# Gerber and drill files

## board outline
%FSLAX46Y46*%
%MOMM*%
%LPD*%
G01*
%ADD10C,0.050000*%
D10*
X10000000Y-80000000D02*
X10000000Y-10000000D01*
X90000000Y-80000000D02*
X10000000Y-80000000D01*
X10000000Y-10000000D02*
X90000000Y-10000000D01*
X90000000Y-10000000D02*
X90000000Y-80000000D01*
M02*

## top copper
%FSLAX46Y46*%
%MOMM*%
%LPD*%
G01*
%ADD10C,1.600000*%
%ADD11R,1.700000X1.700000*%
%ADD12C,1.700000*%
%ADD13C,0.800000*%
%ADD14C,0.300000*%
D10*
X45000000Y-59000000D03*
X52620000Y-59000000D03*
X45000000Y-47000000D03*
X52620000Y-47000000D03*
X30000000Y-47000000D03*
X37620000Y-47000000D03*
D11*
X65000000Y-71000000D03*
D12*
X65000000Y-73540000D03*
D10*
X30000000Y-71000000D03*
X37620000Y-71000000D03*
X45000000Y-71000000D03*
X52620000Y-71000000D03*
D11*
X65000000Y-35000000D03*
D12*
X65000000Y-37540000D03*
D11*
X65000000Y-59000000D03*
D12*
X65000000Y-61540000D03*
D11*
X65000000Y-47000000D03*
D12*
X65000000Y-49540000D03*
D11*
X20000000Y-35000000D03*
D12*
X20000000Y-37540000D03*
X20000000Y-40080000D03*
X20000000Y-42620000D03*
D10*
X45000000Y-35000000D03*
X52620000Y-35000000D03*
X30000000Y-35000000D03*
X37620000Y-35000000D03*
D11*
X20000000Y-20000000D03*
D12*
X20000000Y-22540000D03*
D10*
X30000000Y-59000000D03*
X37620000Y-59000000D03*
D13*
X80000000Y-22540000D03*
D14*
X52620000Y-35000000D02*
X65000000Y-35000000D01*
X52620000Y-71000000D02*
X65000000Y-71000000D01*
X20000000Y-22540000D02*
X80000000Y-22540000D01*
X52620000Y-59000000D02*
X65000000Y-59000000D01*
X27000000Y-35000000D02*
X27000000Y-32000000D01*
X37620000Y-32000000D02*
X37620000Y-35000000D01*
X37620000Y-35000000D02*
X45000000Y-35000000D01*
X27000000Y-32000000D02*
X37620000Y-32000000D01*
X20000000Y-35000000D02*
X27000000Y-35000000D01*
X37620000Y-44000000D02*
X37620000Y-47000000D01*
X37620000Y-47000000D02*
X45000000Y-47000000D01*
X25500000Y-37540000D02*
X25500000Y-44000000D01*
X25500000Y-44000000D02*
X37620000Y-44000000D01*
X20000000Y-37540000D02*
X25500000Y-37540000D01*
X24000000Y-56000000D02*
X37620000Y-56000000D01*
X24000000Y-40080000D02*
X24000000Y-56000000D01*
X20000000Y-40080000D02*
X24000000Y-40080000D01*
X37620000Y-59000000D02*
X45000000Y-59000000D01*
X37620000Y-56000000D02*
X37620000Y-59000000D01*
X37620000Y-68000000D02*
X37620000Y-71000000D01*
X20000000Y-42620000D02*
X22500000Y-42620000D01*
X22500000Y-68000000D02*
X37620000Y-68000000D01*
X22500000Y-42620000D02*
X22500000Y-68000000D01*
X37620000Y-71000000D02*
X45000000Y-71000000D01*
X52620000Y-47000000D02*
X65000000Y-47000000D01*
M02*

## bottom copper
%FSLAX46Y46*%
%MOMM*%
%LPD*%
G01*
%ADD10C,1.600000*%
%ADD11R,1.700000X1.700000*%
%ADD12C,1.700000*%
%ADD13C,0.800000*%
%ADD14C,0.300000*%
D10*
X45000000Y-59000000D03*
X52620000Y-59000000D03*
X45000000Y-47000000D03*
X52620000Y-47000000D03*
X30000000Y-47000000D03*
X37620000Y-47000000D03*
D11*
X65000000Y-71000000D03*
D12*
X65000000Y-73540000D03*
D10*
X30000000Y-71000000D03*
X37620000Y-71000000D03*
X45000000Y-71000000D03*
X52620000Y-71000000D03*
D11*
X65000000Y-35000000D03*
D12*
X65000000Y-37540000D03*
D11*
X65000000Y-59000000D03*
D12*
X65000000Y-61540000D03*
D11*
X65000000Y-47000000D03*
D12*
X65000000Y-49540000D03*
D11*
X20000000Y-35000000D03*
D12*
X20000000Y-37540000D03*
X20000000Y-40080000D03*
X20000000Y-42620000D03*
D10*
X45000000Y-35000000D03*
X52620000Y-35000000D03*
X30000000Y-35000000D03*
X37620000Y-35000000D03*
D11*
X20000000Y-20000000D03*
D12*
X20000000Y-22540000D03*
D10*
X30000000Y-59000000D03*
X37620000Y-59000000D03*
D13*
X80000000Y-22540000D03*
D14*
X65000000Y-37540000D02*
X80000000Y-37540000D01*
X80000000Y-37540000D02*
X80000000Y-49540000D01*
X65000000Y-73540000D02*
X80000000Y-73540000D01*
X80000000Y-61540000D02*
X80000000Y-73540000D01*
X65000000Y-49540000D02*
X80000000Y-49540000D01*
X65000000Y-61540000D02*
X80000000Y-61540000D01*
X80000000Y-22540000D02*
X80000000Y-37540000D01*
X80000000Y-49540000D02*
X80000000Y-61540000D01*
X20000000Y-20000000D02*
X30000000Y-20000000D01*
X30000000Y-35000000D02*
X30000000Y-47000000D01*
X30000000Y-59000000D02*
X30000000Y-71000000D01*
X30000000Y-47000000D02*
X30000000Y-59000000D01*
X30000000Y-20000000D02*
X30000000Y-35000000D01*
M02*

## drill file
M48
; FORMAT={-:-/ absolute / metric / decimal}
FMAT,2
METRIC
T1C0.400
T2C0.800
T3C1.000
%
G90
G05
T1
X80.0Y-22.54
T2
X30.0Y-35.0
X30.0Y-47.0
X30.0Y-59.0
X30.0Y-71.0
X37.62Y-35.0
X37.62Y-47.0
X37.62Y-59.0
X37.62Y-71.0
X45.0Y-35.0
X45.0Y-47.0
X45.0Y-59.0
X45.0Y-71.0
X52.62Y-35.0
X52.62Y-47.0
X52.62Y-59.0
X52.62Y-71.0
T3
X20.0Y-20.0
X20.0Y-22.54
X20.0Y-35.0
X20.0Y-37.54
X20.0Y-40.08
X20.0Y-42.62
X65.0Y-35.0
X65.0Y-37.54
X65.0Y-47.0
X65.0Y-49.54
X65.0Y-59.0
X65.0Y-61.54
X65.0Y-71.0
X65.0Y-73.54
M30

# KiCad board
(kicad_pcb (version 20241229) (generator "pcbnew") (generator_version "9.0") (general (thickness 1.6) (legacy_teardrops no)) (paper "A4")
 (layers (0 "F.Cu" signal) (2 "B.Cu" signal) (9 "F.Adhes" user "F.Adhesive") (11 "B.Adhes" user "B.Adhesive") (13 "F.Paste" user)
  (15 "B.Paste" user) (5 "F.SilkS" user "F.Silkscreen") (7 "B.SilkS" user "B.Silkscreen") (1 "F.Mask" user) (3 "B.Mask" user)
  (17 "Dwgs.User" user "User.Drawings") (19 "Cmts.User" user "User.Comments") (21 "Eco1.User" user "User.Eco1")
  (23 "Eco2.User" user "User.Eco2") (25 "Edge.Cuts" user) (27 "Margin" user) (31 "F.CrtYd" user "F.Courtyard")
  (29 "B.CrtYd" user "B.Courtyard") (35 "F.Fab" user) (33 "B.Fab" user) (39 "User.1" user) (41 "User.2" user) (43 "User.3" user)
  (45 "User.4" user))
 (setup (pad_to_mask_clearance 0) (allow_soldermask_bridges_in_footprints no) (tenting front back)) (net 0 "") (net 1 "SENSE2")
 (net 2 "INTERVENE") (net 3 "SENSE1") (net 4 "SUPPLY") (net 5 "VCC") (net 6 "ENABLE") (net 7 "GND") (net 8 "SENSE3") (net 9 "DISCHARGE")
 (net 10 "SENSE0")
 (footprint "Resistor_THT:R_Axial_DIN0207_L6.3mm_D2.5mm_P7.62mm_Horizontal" (layer "F.Cu") (at 45 59)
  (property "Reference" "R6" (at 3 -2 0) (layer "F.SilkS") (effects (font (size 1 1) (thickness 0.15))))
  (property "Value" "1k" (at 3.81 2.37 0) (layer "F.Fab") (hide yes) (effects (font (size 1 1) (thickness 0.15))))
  (pad "1" thru_hole circle (at 0 0) (size 1.6 1.6) (drill 0.8) (layers "*.Cu" "*.Mask") (remove_unused_layers no) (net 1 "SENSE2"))
  (pad "2" thru_hole circle (at 7.62 0) (size 1.6 1.6) (drill 0.8) (layers "*.Cu" "*.Mask") (remove_unused_layers no) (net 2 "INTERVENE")))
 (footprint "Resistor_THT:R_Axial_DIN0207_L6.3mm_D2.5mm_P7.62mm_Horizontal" (layer "F.Cu") (at 45 47)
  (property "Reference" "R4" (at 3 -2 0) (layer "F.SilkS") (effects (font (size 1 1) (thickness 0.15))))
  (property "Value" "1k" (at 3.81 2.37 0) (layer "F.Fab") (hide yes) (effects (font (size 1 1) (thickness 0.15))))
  (pad "1" thru_hole circle (at 0 0) (size 1.6 1.6) (drill 0.8) (layers "*.Cu" "*.Mask") (remove_unused_layers no) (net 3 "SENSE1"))
  (pad "2" thru_hole circle (at 7.62 0) (size 1.6 1.6) (drill 0.8) (layers "*.Cu" "*.Mask") (remove_unused_layers no) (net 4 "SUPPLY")))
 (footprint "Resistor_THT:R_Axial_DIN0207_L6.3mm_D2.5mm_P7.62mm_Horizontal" (layer "F.Cu") (at 30 47)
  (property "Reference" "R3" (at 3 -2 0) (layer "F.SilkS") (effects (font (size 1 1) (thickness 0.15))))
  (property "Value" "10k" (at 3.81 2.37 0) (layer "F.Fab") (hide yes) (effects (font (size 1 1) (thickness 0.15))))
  (pad "1" thru_hole circle (at 0 0) (size 1.6 1.6) (drill 0.8) (layers "*.Cu" "*.Mask") (remove_unused_layers no) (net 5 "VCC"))
  (pad "2" thru_hole circle (at 7.62 0) (size 1.6 1.6) (drill 0.8) (layers "*.Cu" "*.Mask") (remove_unused_layers no) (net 3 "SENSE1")))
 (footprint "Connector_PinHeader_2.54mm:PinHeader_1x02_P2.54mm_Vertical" (layer "F.Cu") (at 65 71)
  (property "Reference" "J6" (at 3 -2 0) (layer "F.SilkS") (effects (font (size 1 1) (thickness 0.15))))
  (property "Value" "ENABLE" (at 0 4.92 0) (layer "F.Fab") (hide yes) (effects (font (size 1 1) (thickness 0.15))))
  (pad "1" thru_hole rect (at 0 0) (size 1.7 1.7) (drill 1) (layers "*.Cu" "*.Mask") (remove_unused_layers no) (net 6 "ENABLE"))
  (pad "2" thru_hole circle (at 0 2.54) (size 1.7 1.7) (drill 1) (layers "*.Cu" "*.Mask") (remove_unused_layers no) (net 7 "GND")))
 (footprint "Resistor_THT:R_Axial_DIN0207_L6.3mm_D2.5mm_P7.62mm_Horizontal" (layer "F.Cu") (at 30 71)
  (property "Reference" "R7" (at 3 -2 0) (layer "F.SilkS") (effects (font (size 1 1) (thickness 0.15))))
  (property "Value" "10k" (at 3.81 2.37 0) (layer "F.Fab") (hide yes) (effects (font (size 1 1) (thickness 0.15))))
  (pad "1" thru_hole circle (at 0 0) (size 1.6 1.6) (drill 0.8) (layers "*.Cu" "*.Mask") (remove_unused_layers no) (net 5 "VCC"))
  (pad "2" thru_hole circle (at 7.62 0) (size 1.6 1.6) (drill 0.8) (layers "*.Cu" "*.Mask") (remove_unused_layers no) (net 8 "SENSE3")))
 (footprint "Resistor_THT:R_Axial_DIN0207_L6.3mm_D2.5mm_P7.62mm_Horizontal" (layer "F.Cu") (at 45 71)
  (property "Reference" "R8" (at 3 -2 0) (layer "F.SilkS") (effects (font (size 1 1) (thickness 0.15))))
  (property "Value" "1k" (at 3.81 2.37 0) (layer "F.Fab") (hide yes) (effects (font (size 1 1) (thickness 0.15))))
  (pad "1" thru_hole circle (at 0 0) (size 1.6 1.6) (drill 0.8) (layers "*.Cu" "*.Mask") (remove_unused_layers no) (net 8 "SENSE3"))
  (pad "2" thru_hole circle (at 7.62 0) (size 1.6 1.6) (drill 0.8) (layers "*.Cu" "*.Mask") (remove_unused_layers no) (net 6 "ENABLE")))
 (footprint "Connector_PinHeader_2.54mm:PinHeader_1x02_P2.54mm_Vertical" (layer "F.Cu") (at 65 35)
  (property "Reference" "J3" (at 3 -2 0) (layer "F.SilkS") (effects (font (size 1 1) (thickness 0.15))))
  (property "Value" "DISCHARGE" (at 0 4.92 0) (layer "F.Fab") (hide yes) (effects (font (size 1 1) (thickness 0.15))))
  (pad "1" thru_hole rect (at 0 0) (size 1.7 1.7) (drill 1) (layers "*.Cu" "*.Mask") (remove_unused_layers no) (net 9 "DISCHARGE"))
  (pad "2" thru_hole circle (at 0 2.54) (size 1.7 1.7) (drill 1) (layers "*.Cu" "*.Mask") (remove_unused_layers no) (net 7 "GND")))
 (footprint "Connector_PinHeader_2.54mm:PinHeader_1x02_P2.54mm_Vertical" (layer "F.Cu") (at 65 59)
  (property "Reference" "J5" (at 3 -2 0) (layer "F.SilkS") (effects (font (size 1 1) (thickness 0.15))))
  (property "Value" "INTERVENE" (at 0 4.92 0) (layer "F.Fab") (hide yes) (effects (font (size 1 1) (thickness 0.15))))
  (pad "1" thru_hole rect (at 0 0) (size 1.7 1.7) (drill 1) (layers "*.Cu" "*.Mask") (remove_unused_layers no) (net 2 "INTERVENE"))
  (pad "2" thru_hole circle (at 0 2.54) (size 1.7 1.7) (drill 1) (layers "*.Cu" "*.Mask") (remove_unused_layers no) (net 7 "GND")))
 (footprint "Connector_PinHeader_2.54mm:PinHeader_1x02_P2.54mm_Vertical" (layer "F.Cu") (at 65 47)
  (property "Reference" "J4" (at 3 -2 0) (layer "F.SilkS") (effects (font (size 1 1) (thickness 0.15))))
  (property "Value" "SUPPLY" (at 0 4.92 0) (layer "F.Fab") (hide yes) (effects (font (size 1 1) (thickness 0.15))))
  (pad "1" thru_hole rect (at 0 0) (size 1.7 1.7) (drill 1) (layers "*.Cu" "*.Mask") (remove_unused_layers no) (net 4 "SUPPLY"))
  (pad "2" thru_hole circle (at 0 2.54) (size 1.7 1.7) (drill 1) (layers "*.Cu" "*.Mask") (remove_unused_layers no) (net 7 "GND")))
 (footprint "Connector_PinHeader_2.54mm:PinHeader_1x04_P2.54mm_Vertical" (layer "F.Cu") (at 20 35)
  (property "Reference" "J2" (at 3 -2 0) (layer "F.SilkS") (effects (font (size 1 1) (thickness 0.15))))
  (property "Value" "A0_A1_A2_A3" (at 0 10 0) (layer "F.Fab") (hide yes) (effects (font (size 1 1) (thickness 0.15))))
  (pad "1" thru_hole rect (at 0 0) (size 1.7 1.7) (drill 1) (layers "*.Cu" "*.Mask") (remove_unused_layers no) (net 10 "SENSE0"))
  (pad "2" thru_hole circle (at 0 2.54) (size 1.7 1.7) (drill 1) (layers "*.Cu" "*.Mask") (remove_unused_layers no) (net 3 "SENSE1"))
  (pad "3" thru_hole circle (at 0 5.08) (size 1.7 1.7) (drill 1) (layers "*.Cu" "*.Mask") (remove_unused_layers no) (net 1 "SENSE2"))
  (pad "4" thru_hole circle (at 0 7.62) (size 1.7 1.7) (drill 1) (layers "*.Cu" "*.Mask") (remove_unused_layers no) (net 8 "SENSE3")))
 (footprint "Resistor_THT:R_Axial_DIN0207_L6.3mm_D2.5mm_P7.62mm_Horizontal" (layer "F.Cu") (at 45 35)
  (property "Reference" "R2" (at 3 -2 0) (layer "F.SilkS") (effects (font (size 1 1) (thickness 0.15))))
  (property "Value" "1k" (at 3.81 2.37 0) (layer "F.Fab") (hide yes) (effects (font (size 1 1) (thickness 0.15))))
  (pad "1" thru_hole circle (at 0 0) (size 1.6 1.6) (drill 0.8) (layers "*.Cu" "*.Mask") (remove_unused_layers no) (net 10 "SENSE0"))
  (pad "2" thru_hole circle (at 7.62 0) (size 1.6 1.6) (drill 0.8) (layers "*.Cu" "*.Mask") (remove_unused_layers no) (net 9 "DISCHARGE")))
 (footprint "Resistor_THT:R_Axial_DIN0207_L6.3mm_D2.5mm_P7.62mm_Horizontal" (layer "F.Cu") (at 30 35)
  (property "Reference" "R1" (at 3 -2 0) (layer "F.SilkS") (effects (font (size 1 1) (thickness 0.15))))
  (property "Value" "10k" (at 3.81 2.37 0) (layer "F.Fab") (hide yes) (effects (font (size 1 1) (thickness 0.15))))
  (pad "1" thru_hole circle (at 0 0) (size 1.6 1.6) (drill 0.8) (layers "*.Cu" "*.Mask") (remove_unused_layers no) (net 5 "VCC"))
  (pad "2" thru_hole circle (at 7.62 0) (size 1.6 1.6) (drill 0.8) (layers "*.Cu" "*.Mask") (remove_unused_layers no) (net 10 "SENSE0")))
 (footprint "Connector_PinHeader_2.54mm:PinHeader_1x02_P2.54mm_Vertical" (layer "F.Cu") (at 20 20)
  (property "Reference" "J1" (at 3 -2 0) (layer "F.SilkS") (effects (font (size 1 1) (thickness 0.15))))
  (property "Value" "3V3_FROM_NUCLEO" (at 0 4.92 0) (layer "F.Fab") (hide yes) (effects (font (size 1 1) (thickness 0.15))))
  (pad "1" thru_hole rect (at 0 0) (size 1.7 1.7) (drill 1) (layers "*.Cu" "*.Mask") (remove_unused_layers no) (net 5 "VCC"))
  (pad "2" thru_hole circle (at 0 2.54) (size 1.7 1.7) (drill 1) (layers "*.Cu" "*.Mask") (remove_unused_layers no) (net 7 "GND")))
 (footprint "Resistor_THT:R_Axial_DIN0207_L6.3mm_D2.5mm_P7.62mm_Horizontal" (layer "F.Cu") (at 30 59)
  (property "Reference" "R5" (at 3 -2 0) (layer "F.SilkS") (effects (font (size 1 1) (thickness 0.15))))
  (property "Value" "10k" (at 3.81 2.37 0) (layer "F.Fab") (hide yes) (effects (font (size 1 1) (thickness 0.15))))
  (pad "1" thru_hole circle (at 0 0) (size 1.6 1.6) (drill 0.8) (layers "*.Cu" "*.Mask") (remove_unused_layers no) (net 5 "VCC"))
  (pad "2" thru_hole circle (at 7.62 0) (size 1.6 1.6) (drill 0.8) (layers "*.Cu" "*.Mask") (remove_unused_layers no) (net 1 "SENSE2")))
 (gr_line (start 10 80) (end 10 10) (stroke (width 0.05) (type default)) (layer "Edge.Cuts"))
 (gr_line (start 90 80) (end 10 80) (stroke (width 0.05) (type default)) (layer "Edge.Cuts"))
 (gr_line (start 10 10) (end 90 10) (stroke (width 0.05) (type default)) (layer "Edge.Cuts"))
 (gr_line (start 90 10) (end 90 80) (stroke (width 0.05) (type default)) (layer "Edge.Cuts"))
 (segment (start 52.62 35) (end 65 35) (width 0.3) (layer "F.Cu") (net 9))
 (segment (start 52.62 71) (end 65 71) (width 0.3) (layer "F.Cu") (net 6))
 (segment (start 20 22.54) (end 80 22.54) (width 0.3) (layer "F.Cu") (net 7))
 (via (at 80 22.54) (size 0.8) (drill 0.4) (layers "F.Cu" "B.Cu") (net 7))
 (segment (start 65 37.54) (end 80 37.54) (width 0.3) (layer "B.Cu") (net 7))
 (segment (start 80 37.54) (end 80 49.54) (width 0.3) (layer "B.Cu") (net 7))
 (segment (start 65 73.54) (end 80 73.54) (width 0.3) (layer "B.Cu") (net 7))
 (segment (start 80 61.54) (end 80 73.54) (width 0.3) (layer "B.Cu") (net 7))
 (segment (start 65 49.54) (end 80 49.54) (width 0.3) (layer "B.Cu") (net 7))
 (segment (start 65 61.54) (end 80 61.54) (width 0.3) (layer "B.Cu") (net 7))
 (segment (start 80 22.54) (end 80 37.54) (width 0.3) (layer "B.Cu") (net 7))
 (segment (start 80 49.54) (end 80 61.54) (width 0.3) (layer "B.Cu") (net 7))
 (segment (start 52.62 59) (end 65 59) (width 0.3) (layer "F.Cu") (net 2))
 (segment (start 27 35) (end 27 32) (width 0.3) (layer "F.Cu") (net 10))
 (segment (start 37.62 32) (end 37.62 35) (width 0.3) (layer "F.Cu") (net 10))
 (segment (start 37.62 35) (end 45 35) (width 0.3) (layer "F.Cu") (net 10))
 (segment (start 27 32) (end 37.62 32) (width 0.3) (layer "F.Cu") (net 10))
 (segment (start 20 35) (end 27 35) (width 0.3) (layer "F.Cu") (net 10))
 (segment (start 37.62 44) (end 37.62 47) (width 0.3) (layer "F.Cu") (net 3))
 (segment (start 37.62 47) (end 45 47) (width 0.3) (layer "F.Cu") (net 3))
 (segment (start 25.5 37.54) (end 25.5 44) (width 0.3) (layer "F.Cu") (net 3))
 (segment (start 25.5 44) (end 37.62 44) (width 0.3) (layer "F.Cu") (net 3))
 (segment (start 20 37.54) (end 25.5 37.54) (width 0.3) (layer "F.Cu") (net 3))
 (segment (start 24 56) (end 37.62 56) (width 0.3) (layer "F.Cu") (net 1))
 (segment (start 24 40.08) (end 24 56) (width 0.3) (layer "F.Cu") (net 1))
 (segment (start 20 40.08) (end 24 40.08) (width 0.3) (layer "F.Cu") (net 1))
 (segment (start 37.62 59) (end 45 59) (width 0.3) (layer "F.Cu") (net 1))
 (segment (start 37.62 56) (end 37.62 59) (width 0.3) (layer "F.Cu") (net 1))
 (segment (start 37.62 68) (end 37.62 71) (width 0.3) (layer "F.Cu") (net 8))
 (segment (start 20 42.62) (end 22.5 42.62) (width 0.3) (layer "F.Cu") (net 8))
 (segment (start 22.5 68) (end 37.62 68) (width 0.3) (layer "F.Cu") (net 8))
 (segment (start 22.5 42.62) (end 22.5 68) (width 0.3) (layer "F.Cu") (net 8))
 (segment (start 37.62 71) (end 45 71) (width 0.3) (layer "F.Cu") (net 8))
 (segment (start 52.62 47) (end 65 47) (width 0.3) (layer "F.Cu") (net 4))
 (segment (start 20 20) (end 30 20) (width 0.3) (layer "B.Cu") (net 5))
 (segment (start 30 35) (end 30 47) (width 0.3) (layer "B.Cu") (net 5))
 (segment (start 30 59) (end 30 71) (width 0.3) (layer "B.Cu") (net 5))
 (segment (start 30 47) (end 30 59) (width 0.3) (layer "B.Cu") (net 5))
 (segment (start 30 20) (end 30 35) (width 0.3) (layer "B.Cu") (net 5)))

